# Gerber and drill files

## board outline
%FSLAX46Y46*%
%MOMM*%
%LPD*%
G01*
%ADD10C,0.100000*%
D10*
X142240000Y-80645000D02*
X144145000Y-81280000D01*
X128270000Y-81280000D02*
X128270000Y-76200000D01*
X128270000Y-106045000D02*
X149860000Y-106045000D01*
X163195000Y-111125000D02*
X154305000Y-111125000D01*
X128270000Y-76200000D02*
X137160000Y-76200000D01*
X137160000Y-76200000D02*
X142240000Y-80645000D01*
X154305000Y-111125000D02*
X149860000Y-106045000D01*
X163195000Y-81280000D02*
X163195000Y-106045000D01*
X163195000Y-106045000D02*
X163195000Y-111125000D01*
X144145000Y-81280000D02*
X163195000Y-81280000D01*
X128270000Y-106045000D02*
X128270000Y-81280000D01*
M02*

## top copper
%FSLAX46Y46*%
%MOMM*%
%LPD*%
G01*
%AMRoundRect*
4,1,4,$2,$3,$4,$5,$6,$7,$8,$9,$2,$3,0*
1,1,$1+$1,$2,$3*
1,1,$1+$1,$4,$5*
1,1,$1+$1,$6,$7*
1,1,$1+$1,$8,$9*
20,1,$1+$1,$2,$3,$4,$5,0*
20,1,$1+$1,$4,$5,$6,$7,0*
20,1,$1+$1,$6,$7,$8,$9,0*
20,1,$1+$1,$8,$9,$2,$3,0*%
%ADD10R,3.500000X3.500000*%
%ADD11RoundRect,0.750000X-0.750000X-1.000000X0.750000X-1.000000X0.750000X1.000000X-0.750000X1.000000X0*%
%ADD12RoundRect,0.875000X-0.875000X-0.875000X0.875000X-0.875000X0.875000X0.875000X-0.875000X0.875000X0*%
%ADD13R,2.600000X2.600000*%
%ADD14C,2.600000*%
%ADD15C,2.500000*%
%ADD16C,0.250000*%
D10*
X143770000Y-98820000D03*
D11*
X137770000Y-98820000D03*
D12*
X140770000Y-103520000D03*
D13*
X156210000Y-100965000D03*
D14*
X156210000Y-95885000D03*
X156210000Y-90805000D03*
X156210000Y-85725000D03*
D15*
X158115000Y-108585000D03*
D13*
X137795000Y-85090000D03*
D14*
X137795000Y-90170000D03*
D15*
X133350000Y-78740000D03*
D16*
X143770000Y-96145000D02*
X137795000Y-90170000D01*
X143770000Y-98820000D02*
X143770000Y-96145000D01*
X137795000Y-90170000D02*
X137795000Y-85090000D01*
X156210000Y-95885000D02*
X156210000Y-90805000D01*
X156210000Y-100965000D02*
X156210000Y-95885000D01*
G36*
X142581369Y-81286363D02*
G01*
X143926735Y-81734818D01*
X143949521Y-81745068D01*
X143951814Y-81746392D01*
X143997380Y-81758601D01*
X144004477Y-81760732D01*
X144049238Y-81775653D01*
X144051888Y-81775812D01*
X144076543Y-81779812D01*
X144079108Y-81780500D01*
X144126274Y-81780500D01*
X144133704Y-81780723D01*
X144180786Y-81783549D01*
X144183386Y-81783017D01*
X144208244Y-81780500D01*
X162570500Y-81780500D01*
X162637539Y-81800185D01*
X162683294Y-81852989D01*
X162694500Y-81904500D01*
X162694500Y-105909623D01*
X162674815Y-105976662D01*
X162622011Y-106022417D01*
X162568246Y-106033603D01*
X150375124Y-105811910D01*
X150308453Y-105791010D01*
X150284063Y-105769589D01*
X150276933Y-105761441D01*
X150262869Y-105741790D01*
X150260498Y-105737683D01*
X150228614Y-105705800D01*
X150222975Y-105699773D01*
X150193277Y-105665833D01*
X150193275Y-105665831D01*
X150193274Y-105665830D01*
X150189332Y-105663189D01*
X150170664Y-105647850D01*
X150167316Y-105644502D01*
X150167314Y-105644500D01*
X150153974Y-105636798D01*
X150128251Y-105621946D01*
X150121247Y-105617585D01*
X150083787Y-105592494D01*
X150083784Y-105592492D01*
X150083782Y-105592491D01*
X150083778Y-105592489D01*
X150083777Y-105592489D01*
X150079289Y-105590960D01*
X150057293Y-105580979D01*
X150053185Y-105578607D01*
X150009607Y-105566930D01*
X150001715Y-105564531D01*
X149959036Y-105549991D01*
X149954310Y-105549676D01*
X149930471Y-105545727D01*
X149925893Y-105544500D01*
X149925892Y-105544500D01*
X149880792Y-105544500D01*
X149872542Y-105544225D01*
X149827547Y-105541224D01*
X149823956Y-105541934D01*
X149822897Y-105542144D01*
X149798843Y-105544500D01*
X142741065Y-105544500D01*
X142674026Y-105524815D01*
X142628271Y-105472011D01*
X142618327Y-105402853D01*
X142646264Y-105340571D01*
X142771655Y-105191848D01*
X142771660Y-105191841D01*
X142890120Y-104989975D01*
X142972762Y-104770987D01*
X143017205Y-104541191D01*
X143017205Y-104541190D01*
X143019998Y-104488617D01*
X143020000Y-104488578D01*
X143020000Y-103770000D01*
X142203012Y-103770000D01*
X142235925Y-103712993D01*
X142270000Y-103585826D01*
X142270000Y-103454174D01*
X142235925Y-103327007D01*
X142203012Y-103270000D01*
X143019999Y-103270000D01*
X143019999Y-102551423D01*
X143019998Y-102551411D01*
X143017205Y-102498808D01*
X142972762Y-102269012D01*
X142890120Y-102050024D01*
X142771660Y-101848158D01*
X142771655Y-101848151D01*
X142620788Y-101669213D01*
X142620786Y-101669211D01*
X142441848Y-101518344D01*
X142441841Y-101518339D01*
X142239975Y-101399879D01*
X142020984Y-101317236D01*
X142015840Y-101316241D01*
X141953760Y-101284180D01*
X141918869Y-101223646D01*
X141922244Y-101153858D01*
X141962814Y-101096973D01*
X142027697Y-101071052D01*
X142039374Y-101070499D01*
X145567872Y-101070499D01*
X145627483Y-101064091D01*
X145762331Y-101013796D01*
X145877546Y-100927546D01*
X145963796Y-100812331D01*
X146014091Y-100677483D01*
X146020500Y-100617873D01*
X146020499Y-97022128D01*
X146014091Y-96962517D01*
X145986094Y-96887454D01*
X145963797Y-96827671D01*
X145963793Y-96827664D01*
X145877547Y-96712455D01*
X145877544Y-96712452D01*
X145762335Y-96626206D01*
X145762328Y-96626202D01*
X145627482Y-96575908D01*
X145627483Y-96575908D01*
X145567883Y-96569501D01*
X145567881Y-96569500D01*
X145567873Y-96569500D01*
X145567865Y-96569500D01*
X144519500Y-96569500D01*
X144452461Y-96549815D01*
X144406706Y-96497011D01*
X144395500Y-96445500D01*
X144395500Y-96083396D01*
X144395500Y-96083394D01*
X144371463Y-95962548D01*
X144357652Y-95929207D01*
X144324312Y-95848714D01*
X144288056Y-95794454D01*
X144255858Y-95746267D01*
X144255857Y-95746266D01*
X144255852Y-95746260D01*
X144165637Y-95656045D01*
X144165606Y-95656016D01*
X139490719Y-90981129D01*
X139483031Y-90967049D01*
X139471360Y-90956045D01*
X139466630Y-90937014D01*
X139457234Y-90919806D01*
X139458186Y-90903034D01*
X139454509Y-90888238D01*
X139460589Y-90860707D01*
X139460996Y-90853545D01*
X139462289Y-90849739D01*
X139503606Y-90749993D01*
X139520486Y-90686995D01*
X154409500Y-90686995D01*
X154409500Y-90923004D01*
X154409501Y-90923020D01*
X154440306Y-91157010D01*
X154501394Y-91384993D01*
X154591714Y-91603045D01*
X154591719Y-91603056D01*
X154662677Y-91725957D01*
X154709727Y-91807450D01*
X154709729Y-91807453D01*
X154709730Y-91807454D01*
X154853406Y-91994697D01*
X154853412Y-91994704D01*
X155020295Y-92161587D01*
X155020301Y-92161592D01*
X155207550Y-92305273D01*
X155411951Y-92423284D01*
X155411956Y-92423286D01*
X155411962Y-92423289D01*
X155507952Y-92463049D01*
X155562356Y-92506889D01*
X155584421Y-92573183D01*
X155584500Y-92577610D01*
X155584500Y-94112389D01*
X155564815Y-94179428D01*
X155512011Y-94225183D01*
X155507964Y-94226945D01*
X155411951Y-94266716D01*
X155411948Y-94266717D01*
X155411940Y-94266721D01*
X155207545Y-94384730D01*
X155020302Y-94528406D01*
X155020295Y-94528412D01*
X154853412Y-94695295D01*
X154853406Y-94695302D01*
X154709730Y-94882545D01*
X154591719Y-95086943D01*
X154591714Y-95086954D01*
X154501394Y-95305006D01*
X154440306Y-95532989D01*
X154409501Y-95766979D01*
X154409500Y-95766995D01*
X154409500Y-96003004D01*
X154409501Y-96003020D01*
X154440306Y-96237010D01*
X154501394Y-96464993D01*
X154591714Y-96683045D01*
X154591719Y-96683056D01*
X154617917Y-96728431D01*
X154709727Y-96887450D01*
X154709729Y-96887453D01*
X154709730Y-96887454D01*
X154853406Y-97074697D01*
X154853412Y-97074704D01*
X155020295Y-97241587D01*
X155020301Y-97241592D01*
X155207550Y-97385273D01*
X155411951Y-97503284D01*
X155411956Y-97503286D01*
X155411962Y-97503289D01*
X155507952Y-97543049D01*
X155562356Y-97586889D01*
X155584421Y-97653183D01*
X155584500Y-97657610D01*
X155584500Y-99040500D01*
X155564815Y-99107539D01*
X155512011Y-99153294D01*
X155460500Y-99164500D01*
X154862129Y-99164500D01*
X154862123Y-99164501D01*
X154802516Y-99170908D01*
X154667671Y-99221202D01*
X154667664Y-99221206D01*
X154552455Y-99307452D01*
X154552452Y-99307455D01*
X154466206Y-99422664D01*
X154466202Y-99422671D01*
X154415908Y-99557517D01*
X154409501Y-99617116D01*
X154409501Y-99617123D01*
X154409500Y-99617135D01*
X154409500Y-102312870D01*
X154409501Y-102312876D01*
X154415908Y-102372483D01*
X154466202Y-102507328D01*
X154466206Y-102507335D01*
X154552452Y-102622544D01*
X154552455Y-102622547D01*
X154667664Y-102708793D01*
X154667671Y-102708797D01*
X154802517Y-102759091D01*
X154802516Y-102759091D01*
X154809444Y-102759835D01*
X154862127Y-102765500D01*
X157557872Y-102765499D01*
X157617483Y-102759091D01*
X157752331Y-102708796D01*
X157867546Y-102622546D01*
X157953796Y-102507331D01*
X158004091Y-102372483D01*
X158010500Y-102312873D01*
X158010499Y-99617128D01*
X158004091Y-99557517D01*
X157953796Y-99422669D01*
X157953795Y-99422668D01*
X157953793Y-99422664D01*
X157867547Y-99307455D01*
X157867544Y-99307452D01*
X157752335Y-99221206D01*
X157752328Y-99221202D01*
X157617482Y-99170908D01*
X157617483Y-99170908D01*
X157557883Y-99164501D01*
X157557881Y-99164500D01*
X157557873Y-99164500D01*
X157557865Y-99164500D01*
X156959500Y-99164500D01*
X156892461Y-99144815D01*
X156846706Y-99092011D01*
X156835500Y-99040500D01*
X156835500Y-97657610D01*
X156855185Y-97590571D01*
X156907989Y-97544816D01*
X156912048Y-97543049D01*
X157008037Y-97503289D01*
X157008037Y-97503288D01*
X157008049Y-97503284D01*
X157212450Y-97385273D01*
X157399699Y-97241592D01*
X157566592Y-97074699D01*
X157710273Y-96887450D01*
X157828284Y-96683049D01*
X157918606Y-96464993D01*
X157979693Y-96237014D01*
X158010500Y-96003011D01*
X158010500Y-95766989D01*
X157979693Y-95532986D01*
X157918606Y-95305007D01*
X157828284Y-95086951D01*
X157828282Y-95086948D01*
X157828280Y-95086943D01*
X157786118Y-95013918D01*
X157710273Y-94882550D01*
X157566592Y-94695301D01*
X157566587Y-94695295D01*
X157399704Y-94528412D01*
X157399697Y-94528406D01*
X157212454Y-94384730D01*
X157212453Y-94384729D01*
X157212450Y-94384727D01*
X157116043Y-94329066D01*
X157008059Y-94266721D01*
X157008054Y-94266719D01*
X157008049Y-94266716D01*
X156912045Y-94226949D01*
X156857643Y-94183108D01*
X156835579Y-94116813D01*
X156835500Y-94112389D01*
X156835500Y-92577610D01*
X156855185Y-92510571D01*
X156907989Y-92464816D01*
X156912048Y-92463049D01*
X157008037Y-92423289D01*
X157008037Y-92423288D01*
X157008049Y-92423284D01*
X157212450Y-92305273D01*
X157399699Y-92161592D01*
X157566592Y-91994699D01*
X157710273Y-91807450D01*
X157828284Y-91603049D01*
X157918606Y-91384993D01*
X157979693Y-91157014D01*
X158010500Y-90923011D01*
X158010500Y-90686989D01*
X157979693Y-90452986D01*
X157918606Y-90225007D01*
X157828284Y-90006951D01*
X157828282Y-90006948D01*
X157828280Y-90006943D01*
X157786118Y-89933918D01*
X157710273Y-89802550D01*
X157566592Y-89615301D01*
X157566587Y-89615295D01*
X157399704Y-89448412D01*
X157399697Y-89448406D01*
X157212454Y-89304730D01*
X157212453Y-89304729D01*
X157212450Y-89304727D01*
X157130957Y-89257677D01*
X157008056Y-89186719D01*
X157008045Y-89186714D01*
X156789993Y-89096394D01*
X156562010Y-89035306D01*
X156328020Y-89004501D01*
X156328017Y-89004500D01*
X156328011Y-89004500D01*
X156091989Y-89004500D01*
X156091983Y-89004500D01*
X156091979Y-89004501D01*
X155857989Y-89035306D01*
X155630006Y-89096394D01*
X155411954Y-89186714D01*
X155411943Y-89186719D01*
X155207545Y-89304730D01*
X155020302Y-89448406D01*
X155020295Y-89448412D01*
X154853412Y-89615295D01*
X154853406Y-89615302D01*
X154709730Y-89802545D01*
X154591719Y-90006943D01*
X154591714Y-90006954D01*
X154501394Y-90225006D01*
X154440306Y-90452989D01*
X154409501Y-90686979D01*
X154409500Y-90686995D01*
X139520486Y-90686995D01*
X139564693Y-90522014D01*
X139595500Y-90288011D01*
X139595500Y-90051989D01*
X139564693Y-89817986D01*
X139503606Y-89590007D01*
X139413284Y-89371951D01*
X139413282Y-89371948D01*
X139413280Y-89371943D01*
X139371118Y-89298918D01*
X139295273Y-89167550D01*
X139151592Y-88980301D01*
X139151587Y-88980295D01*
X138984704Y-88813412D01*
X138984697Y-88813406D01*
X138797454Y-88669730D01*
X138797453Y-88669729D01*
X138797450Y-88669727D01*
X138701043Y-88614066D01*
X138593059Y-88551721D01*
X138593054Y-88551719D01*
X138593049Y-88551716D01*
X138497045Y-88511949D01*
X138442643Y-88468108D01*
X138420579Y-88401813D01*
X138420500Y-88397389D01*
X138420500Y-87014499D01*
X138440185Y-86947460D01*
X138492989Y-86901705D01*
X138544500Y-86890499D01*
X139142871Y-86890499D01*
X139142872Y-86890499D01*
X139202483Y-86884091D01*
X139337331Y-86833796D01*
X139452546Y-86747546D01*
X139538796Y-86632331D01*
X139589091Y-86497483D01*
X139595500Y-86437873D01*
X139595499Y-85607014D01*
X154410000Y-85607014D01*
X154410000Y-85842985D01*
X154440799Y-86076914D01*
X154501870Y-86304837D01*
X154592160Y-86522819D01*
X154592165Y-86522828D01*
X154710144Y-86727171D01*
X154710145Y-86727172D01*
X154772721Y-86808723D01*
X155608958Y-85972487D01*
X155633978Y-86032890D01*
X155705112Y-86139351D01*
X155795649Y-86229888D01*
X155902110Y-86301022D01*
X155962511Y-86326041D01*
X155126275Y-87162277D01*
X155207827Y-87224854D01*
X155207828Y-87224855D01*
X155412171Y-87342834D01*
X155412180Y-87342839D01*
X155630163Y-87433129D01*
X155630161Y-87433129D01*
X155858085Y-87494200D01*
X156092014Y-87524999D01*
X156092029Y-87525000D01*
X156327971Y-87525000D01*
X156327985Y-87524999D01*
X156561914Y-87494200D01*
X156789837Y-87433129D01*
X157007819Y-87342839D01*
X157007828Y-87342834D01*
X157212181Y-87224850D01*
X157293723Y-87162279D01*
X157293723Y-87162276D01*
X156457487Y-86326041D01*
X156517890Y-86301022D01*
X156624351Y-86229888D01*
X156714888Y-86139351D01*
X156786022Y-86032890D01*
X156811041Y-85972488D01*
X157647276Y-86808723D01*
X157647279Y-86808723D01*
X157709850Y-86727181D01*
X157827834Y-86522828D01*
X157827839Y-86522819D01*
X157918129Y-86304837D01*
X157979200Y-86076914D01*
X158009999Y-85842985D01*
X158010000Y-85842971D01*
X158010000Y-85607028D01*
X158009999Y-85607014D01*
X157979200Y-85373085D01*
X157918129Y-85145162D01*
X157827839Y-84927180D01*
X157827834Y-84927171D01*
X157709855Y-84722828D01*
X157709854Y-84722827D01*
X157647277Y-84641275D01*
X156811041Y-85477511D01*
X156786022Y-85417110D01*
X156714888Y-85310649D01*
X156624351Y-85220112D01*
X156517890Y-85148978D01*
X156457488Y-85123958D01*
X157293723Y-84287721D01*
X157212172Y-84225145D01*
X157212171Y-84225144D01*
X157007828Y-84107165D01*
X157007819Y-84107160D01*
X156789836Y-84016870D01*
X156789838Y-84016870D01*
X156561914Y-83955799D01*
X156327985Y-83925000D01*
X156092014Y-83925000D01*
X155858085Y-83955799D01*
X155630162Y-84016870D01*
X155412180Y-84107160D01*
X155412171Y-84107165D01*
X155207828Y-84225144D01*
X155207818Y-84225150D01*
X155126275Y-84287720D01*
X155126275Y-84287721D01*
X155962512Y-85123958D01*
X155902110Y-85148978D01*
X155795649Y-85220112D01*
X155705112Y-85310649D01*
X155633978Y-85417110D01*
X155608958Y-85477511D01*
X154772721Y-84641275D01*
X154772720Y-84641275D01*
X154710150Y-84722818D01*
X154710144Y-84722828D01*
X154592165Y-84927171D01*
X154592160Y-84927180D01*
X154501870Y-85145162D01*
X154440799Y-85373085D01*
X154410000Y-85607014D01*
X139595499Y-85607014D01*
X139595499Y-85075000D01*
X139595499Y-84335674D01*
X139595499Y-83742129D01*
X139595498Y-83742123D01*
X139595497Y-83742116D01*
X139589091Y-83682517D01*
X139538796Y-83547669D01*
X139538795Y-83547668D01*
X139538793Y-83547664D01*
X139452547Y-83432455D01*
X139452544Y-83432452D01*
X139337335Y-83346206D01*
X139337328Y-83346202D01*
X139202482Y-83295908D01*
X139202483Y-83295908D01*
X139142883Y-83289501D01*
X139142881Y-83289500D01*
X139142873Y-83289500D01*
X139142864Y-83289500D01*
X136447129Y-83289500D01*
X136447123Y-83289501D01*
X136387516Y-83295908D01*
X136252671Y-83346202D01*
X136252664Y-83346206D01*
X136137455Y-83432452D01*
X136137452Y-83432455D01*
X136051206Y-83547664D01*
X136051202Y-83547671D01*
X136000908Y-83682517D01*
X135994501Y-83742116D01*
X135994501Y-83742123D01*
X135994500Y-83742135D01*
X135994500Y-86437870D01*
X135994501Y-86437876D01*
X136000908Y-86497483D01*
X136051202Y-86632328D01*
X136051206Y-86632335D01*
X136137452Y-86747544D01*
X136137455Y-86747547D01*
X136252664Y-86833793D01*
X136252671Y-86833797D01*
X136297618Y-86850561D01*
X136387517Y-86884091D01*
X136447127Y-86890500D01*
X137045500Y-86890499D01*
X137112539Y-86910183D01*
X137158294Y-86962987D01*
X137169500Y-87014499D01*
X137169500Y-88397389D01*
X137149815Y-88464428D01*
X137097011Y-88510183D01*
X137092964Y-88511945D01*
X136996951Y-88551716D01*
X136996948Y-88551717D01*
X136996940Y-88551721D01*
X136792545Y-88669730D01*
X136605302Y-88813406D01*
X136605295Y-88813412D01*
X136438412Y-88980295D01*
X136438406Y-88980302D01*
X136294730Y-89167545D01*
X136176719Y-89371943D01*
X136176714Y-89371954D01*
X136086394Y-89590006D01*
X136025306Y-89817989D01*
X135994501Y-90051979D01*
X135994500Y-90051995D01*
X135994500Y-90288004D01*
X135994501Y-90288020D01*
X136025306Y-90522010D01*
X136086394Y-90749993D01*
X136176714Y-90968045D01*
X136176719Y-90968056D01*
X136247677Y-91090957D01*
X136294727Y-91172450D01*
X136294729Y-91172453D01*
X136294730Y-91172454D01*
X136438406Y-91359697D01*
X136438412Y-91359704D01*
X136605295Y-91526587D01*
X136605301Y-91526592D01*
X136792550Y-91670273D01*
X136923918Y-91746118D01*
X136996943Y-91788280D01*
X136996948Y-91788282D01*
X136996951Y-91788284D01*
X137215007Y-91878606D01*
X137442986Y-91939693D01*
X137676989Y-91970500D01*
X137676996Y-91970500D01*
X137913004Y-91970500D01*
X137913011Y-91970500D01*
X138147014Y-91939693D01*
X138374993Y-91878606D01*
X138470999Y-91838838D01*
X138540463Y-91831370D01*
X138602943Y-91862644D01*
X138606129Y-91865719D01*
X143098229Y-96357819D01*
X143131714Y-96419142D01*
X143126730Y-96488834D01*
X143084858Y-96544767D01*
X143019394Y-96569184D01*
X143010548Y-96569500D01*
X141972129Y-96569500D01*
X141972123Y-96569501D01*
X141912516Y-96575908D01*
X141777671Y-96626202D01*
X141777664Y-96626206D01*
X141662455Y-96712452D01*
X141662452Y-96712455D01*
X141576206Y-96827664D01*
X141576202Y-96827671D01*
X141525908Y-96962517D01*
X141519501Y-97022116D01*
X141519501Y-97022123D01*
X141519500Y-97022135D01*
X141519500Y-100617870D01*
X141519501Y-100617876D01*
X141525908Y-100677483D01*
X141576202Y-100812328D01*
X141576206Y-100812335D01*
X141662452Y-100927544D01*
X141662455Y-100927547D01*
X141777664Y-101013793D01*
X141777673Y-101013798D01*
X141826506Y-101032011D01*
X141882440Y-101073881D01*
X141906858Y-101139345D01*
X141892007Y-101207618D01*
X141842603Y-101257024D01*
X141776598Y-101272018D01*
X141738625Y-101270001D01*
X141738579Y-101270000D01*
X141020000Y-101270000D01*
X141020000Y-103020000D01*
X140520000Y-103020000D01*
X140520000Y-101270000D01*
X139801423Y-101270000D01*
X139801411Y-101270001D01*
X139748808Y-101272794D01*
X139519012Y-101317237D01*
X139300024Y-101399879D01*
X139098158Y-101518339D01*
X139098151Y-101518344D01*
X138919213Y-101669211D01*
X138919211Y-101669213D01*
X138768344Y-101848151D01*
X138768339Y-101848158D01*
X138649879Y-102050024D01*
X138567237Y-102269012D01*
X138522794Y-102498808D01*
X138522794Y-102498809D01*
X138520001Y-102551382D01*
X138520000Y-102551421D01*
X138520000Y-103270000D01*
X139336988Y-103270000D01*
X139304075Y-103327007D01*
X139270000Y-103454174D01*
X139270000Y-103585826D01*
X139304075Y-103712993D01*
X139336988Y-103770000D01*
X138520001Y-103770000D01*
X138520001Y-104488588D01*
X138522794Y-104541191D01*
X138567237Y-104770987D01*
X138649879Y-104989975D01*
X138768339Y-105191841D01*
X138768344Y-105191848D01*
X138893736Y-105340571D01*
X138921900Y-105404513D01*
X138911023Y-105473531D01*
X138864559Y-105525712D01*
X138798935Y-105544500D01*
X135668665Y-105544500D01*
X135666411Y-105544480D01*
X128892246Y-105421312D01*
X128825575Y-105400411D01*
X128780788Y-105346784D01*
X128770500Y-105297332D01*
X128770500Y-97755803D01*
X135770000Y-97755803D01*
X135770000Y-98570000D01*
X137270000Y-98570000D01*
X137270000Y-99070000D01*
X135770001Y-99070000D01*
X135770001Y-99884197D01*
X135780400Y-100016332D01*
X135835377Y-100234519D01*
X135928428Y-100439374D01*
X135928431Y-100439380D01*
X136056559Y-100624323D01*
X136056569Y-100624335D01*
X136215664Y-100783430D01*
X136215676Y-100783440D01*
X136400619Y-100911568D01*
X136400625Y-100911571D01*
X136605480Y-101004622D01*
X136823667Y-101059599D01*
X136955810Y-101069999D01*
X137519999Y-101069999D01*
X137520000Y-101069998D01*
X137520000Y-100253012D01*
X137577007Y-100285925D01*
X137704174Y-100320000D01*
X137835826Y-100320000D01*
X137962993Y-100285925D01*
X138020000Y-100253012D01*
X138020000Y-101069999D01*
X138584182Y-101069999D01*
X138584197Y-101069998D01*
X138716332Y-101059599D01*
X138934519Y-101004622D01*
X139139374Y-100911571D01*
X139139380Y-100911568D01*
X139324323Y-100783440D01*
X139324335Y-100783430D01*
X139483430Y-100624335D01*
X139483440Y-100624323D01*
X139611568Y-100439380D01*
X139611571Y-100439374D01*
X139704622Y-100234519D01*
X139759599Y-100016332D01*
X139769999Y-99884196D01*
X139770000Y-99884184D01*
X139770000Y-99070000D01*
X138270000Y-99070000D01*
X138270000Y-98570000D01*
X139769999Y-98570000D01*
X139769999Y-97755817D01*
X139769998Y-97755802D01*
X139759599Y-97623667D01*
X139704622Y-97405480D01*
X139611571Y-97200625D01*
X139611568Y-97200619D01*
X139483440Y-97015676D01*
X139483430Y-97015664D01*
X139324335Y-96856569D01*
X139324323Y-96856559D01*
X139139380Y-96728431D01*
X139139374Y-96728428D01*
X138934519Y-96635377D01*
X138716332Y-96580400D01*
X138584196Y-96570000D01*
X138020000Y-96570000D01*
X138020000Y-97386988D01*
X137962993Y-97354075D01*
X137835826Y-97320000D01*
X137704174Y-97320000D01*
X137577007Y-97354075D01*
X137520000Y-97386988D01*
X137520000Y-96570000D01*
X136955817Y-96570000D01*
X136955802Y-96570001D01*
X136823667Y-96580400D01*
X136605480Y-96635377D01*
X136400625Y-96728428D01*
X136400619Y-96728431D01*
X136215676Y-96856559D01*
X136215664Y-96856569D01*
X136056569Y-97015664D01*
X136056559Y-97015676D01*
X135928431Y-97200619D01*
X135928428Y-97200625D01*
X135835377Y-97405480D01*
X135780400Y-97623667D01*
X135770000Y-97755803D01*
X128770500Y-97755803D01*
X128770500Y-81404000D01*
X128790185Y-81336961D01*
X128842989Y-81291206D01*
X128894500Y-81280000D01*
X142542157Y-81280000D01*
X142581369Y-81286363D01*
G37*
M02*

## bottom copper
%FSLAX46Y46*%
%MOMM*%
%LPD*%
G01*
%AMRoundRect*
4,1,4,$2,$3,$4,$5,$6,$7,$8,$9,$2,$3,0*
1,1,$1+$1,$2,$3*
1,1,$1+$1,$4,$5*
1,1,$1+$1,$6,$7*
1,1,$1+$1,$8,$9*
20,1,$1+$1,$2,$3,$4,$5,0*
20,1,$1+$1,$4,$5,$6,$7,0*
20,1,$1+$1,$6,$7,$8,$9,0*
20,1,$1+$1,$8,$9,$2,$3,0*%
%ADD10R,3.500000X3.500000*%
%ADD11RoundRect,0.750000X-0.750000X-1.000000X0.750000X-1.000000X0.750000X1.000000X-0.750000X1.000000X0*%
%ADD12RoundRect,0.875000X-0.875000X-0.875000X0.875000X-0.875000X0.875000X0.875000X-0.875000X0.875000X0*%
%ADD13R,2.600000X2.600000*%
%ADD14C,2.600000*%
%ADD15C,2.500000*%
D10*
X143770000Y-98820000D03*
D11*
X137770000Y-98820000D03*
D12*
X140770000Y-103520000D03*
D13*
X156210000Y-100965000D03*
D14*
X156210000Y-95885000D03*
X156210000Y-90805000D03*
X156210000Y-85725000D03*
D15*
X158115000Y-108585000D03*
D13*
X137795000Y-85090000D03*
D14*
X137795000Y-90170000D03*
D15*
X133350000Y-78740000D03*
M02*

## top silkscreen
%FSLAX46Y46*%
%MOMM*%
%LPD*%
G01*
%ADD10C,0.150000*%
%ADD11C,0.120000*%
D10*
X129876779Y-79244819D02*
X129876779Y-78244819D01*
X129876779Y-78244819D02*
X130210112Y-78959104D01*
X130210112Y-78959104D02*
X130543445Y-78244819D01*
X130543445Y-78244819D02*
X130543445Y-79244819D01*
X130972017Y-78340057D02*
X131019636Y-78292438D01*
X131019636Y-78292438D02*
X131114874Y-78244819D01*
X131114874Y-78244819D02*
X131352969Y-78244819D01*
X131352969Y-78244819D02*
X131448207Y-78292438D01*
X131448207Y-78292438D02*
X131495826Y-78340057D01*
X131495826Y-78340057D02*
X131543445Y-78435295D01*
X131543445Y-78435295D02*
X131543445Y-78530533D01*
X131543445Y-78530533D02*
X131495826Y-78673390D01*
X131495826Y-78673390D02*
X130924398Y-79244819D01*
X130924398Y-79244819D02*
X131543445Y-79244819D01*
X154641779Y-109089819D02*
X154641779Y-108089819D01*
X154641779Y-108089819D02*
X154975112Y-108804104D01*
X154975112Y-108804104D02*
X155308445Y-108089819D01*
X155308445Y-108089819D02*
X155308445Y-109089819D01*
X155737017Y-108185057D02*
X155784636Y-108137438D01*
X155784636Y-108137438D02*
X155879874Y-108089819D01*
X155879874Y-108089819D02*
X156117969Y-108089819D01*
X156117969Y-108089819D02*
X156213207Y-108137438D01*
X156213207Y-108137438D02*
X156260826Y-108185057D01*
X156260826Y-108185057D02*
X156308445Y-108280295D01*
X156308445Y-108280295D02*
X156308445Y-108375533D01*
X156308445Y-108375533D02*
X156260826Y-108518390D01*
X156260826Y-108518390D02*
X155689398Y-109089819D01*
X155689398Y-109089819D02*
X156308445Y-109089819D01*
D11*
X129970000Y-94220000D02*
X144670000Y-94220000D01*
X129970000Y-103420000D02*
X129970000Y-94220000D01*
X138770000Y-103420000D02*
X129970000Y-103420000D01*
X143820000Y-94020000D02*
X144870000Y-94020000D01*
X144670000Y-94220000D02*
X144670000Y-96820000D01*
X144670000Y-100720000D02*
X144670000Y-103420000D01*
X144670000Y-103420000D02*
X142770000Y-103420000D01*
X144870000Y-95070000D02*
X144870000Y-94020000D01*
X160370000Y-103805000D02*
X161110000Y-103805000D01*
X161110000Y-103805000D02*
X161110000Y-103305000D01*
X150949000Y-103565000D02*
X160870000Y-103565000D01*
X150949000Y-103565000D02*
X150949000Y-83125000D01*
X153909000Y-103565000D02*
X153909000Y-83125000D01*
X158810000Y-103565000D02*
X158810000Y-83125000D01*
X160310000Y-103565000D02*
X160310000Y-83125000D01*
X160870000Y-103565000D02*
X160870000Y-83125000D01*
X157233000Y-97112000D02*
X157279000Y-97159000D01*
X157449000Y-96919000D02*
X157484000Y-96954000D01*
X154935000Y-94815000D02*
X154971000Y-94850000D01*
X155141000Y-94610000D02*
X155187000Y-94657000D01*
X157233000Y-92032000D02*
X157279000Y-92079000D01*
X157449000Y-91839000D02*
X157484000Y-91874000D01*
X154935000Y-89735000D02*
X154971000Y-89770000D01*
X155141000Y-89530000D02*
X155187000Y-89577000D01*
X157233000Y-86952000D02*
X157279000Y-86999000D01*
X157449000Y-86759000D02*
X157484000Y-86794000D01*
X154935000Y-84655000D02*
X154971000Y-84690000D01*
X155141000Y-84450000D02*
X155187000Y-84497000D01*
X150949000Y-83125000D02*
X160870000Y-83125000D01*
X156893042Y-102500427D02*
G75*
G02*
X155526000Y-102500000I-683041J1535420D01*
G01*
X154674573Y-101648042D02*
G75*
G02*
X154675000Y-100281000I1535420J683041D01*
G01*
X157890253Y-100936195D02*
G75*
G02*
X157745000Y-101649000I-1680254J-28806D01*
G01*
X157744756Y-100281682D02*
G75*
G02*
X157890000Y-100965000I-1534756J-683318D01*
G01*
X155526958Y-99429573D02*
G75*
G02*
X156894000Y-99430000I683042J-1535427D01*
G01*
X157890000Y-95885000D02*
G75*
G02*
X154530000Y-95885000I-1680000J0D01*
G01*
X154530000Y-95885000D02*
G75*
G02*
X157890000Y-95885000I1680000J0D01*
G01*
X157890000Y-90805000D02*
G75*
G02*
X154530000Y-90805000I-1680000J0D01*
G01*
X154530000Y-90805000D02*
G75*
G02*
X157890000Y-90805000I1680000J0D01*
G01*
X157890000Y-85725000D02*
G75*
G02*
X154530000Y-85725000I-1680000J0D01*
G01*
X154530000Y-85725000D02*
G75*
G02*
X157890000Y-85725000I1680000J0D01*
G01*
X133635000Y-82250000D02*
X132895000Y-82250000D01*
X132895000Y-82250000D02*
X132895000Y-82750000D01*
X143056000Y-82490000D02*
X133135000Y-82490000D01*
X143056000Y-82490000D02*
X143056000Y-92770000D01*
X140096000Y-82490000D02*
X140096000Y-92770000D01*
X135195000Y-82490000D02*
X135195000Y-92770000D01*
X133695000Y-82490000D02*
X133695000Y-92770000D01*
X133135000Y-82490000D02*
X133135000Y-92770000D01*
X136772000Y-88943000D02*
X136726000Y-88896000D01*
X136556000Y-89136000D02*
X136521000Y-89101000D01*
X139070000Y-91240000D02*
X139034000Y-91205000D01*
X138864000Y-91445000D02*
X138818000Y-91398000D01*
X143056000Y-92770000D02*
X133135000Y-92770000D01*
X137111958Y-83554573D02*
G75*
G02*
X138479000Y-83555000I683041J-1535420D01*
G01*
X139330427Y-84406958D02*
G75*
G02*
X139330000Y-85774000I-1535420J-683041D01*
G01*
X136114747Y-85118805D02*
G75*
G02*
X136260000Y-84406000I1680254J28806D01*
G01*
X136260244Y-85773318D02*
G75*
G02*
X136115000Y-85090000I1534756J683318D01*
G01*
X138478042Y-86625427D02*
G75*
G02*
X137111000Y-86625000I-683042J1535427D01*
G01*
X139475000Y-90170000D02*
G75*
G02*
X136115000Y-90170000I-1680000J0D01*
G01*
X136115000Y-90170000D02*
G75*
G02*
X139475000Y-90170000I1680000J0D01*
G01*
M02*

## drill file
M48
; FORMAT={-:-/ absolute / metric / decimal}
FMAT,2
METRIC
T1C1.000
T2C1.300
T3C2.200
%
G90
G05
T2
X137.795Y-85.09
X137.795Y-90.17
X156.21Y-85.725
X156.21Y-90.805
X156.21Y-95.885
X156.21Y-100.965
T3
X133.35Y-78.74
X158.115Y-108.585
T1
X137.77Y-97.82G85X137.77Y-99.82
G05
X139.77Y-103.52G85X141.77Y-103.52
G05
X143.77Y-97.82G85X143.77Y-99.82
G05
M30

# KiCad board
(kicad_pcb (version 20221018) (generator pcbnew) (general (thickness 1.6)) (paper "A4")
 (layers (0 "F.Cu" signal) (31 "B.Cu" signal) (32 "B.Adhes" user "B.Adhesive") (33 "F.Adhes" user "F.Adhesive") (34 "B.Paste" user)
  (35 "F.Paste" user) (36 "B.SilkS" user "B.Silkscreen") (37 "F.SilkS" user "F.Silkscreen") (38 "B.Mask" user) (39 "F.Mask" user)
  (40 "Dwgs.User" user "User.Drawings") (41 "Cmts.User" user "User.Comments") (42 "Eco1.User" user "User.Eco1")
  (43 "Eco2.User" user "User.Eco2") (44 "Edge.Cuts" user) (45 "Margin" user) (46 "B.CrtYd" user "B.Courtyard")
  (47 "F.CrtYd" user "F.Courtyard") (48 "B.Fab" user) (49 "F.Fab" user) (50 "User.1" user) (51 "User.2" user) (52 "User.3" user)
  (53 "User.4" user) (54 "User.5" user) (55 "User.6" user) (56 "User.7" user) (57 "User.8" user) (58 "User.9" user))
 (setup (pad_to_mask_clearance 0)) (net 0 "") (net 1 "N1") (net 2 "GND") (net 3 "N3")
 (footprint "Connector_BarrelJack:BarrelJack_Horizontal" (layer "F.Cu") (at 143.77 98.82)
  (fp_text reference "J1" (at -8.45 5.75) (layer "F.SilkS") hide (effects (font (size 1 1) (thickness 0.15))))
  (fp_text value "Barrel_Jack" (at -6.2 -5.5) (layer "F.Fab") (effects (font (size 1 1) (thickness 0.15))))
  (fp_line (start -13.8 -4.6) (end 0.9 -4.6) (stroke (width 0.12) (type solid)) (layer "F.SilkS"))
  (fp_line (start -13.8 4.6) (end -13.8 -4.6) (stroke (width 0.12) (type solid)) (layer "F.SilkS"))
  (fp_line (start -5 4.6) (end -13.8 4.6) (stroke (width 0.12) (type solid)) (layer "F.SilkS"))
  (fp_line (start 0.05 -4.8) (end 1.1 -4.8) (stroke (width 0.12) (type solid)) (layer "F.SilkS"))
  (fp_line (start 0.9 -4.6) (end 0.9 -2) (stroke (width 0.12) (type solid)) (layer "F.SilkS"))
  (fp_line (start 0.9 1.9) (end 0.9 4.6) (stroke (width 0.12) (type solid)) (layer "F.SilkS"))
  (fp_line (start 0.9 4.6) (end -1 4.6) (stroke (width 0.12) (type solid)) (layer "F.SilkS"))
  (fp_line (start 1.1 -3.75) (end 1.1 -4.8) (stroke (width 0.12) (type solid)) (layer "F.SilkS"))
  (pad "1" thru_hole rect (at 0 0) (size 3.5 3.5) (drill oval 1 3) (layers "*.Cu" "*.Mask") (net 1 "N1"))
  (pad "2" thru_hole roundrect (at -6 0) (size 3 3.5) (drill oval 1 3) (layers "*.Cu" "*.Mask") (roundrect_rratio 0.25) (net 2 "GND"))
  (pad "3" thru_hole roundrect (at -3 4.7) (size 3.5 3.5) (drill oval 3 1) (layers "*.Cu" "*.Mask") (roundrect_rratio 0.25) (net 2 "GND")))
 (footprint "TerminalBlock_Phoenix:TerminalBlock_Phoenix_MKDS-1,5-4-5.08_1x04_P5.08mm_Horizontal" (layer "F.Cu") (at 156.21 100.965 90)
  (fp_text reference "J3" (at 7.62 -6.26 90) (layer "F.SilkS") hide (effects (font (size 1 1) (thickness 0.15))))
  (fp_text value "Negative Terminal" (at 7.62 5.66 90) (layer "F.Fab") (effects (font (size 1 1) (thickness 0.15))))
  (fp_line (start -2.84 4.16) (end -2.84 4.9) (stroke (width 0.12) (type solid)) (layer "F.SilkS"))
  (fp_line (start -2.84 4.9) (end -2.34 4.9) (stroke (width 0.12) (type solid)) (layer "F.SilkS"))
  (fp_line (start -2.6 -5.261) (end -2.6 4.66) (stroke (width 0.12) (type solid)) (layer "F.SilkS"))
  (fp_line (start -2.6 -5.261) (end 17.84 -5.261) (stroke (width 0.12) (type solid)) (layer "F.SilkS"))
  (fp_line (start -2.6 -2.301) (end 17.84 -2.301) (stroke (width 0.12) (type solid)) (layer "F.SilkS"))
  (fp_line (start -2.6 2.6) (end 17.84 2.6) (stroke (width 0.12) (type solid)) (layer "F.SilkS"))
  (fp_line (start -2.6 4.1) (end 17.84 4.1) (stroke (width 0.12) (type solid)) (layer "F.SilkS"))
  (fp_line (start -2.6 4.66) (end 17.84 4.66) (stroke (width 0.12) (type solid)) (layer "F.SilkS"))
  (fp_line (start 3.853 1.023) (end 3.806 1.069) (stroke (width 0.12) (type solid)) (layer "F.SilkS"))
  (fp_line (start 4.046 1.239) (end 4.011 1.274) (stroke (width 0.12) (type solid)) (layer "F.SilkS"))
  (fp_line (start 6.15 -1.275) (end 6.115 -1.239) (stroke (width 0.12) (type solid)) (layer "F.SilkS"))
  (fp_line (start 6.355 -1.069) (end 6.308 -1.023) (stroke (width 0.12) (type solid)) (layer "F.SilkS"))
  (fp_line (start 8.933 1.023) (end 8.886 1.069) (stroke (width 0.12) (type solid)) (layer "F.SilkS"))
  (fp_line (start 9.126 1.239) (end 9.091 1.274) (stroke (width 0.12) (type solid)) (layer "F.SilkS"))
  (fp_line (start 11.23 -1.275) (end 11.195 -1.239) (stroke (width 0.12) (type solid)) (layer "F.SilkS"))
  (fp_line (start 11.435 -1.069) (end 11.388 -1.023) (stroke (width 0.12) (type solid)) (layer "F.SilkS"))
  (fp_line (start 14.013 1.023) (end 13.966 1.069) (stroke (width 0.12) (type solid)) (layer "F.SilkS"))
  (fp_line (start 14.206 1.239) (end 14.171 1.274) (stroke (width 0.12) (type solid)) (layer "F.SilkS"))
  (fp_line (start 16.31 -1.275) (end 16.275 -1.239) (stroke (width 0.12) (type solid)) (layer "F.SilkS"))
  (fp_line (start 16.515 -1.069) (end 16.468 -1.023) (stroke (width 0.12) (type solid)) (layer "F.SilkS"))
  (fp_line (start 17.84 -5.261) (end 17.84 4.66) (stroke (width 0.12) (type solid)) (layer "F.SilkS"))
  (fp_arc (start -1.535427 0.683042) (mid -1.680501 -0.000524) (end -1.535 -0.684) (stroke (width 0.12) (type solid)) (layer "F.SilkS"))
  (fp_arc (start -0.683042 -1.535427) (mid 0.000524 -1.680501) (end 0.684 -1.535) (stroke (width 0.12) (type solid)) (layer "F.SilkS"))
  (fp_arc (start 0.028805 1.680253) (mid -0.335551 1.646659) (end -0.684 1.535) (stroke (width 0.12) (type solid)) (layer "F.SilkS"))
  (fp_arc (start 0.683318 1.534756) (mid 0.349292 1.643288) (end 0 1.68) (stroke (width 0.12) (type solid)) (layer "F.SilkS"))
  (fp_arc (start 1.535427 -0.683042) (mid 1.680501 0.000524) (end 1.535 0.684) (stroke (width 0.12) (type solid)) (layer "F.SilkS"))
  (fp_circle (center 5.08 0) (end 6.76 0) (stroke (width 0.12) (type solid)) (fill none) (layer "F.SilkS"))
  (fp_circle (center 10.16 0) (end 11.84 0) (stroke (width 0.12) (type solid)) (fill none) (layer "F.SilkS"))
  (fp_circle (center 15.24 0) (end 16.92 0) (stroke (width 0.12) (type solid)) (fill none) (layer "F.SilkS"))
  (pad "1" thru_hole rect (at 0 0 90) (size 2.6 2.6) (drill 1.3) (layers "*.Cu" "*.Mask") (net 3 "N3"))
  (pad "2" thru_hole circle (at 5.08 0 90) (size 2.6 2.6) (drill 1.3) (layers "*.Cu" "*.Mask") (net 3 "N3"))
  (pad "3" thru_hole circle (at 10.16 0 90) (size 2.6 2.6) (drill 1.3) (layers "*.Cu" "*.Mask") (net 3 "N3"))
  (pad "4" thru_hole circle (at 15.24 0 90) (size 2.6 2.6) (drill 1.3) (layers "*.Cu" "*.Mask") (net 2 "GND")))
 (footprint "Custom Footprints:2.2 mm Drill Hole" (layer "F.Cu") (at 158.115 108.585)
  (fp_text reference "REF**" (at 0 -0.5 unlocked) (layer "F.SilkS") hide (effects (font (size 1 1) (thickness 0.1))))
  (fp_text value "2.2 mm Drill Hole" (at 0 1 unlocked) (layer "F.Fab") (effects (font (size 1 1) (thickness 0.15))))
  (pad "" np_thru_hole circle (at 0 0) (size 2.5 2.5) (drill 2.2) (layers "F&B.Cu" "*.Mask")))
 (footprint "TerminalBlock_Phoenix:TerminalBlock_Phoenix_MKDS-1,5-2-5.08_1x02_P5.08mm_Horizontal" (layer "F.Cu") (at 137.795 85.09 -90)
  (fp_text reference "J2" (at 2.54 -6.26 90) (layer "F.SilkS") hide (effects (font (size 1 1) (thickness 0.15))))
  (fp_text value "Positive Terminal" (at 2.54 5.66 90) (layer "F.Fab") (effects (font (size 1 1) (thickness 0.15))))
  (fp_line (start -2.84 4.16) (end -2.84 4.9) (stroke (width 0.12) (type solid)) (layer "F.SilkS"))
  (fp_line (start -2.84 4.9) (end -2.34 4.9) (stroke (width 0.12) (type solid)) (layer "F.SilkS"))
  (fp_line (start -2.6 -5.261) (end -2.6 4.66) (stroke (width 0.12) (type solid)) (layer "F.SilkS"))
  (fp_line (start -2.6 -5.261) (end 7.68 -5.261) (stroke (width 0.12) (type solid)) (layer "F.SilkS"))
  (fp_line (start -2.6 -2.301) (end 7.68 -2.301) (stroke (width 0.12) (type solid)) (layer "F.SilkS"))
  (fp_line (start -2.6 2.6) (end 7.68 2.6) (stroke (width 0.12) (type solid)) (layer "F.SilkS"))
  (fp_line (start -2.6 4.1) (end 7.68 4.1) (stroke (width 0.12) (type solid)) (layer "F.SilkS"))
  (fp_line (start -2.6 4.66) (end 7.68 4.66) (stroke (width 0.12) (type solid)) (layer "F.SilkS"))
  (fp_line (start 3.853 1.023) (end 3.806 1.069) (stroke (width 0.12) (type solid)) (layer "F.SilkS"))
  (fp_line (start 4.046 1.239) (end 4.011 1.274) (stroke (width 0.12) (type solid)) (layer "F.SilkS"))
  (fp_line (start 6.15 -1.275) (end 6.115 -1.239) (stroke (width 0.12) (type solid)) (layer "F.SilkS"))
  (fp_line (start 6.355 -1.069) (end 6.308 -1.023) (stroke (width 0.12) (type solid)) (layer "F.SilkS"))
  (fp_line (start 7.68 -5.261) (end 7.68 4.66) (stroke (width 0.12) (type solid)) (layer "F.SilkS"))
  (fp_arc (start -1.535427 0.683042) (mid -1.680501 -0.000524) (end -1.535 -0.684) (stroke (width 0.12) (type solid)) (layer "F.SilkS"))
  (fp_arc (start -0.683042 -1.535427) (mid 0.000524 -1.680501) (end 0.684 -1.535) (stroke (width 0.12) (type solid)) (layer "F.SilkS"))
  (fp_arc (start 0.028805 1.680253) (mid -0.335551 1.646659) (end -0.684 1.535) (stroke (width 0.12) (type solid)) (layer "F.SilkS"))
  (fp_arc (start 0.683318 1.534756) (mid 0.349292 1.643288) (end 0 1.68) (stroke (width 0.12) (type solid)) (layer "F.SilkS"))
  (fp_arc (start 1.535427 -0.683042) (mid 1.680501 0.000524) (end 1.535 0.684) (stroke (width 0.12) (type solid)) (layer "F.SilkS"))
  (fp_circle (center 5.08 0) (end 6.76 0) (stroke (width 0.12) (type solid)) (fill none) (layer "F.SilkS"))
  (pad "1" thru_hole rect (at 0 0 270) (size 2.6 2.6) (drill 1.3) (layers "*.Cu" "*.Mask") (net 1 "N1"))
  (pad "2" thru_hole circle (at 5.08 0 270) (size 2.6 2.6) (drill 1.3) (layers "*.Cu" "*.Mask") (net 1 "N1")))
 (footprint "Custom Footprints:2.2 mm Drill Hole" (layer "F.Cu") (at 133.35 78.74)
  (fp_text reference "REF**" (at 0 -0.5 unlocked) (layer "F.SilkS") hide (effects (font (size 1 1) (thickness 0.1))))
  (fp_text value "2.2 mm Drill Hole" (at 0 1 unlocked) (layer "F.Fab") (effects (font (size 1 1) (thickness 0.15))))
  (pad "" np_thru_hole circle (at 0 0) (size 2.5 2.5) (drill 2.2) (layers "F&B.Cu" "*.Mask")))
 (gr_line (start 142.24 80.645) (end 144.145 81.28) (stroke (width 0.1) (type default)) (layer "Edge.Cuts"))
 (gr_line (start 128.27 81.28) (end 128.27 76.2) (stroke (width 0.1) (type default)) (layer "Edge.Cuts"))
 (gr_line (start 128.27 106.045) (end 149.86 106.045) (stroke (width 0.1) (type default)) (layer "Edge.Cuts"))
 (gr_line (start 163.195 111.125) (end 154.305 111.125) (stroke (width 0.1) (type default)) (layer "Edge.Cuts"))
 (gr_line (start 128.27 76.2) (end 137.16 76.2) (stroke (width 0.1) (type default)) (layer "Edge.Cuts"))
 (gr_line (start 137.16 76.2) (end 142.24 80.645) (stroke (width 0.1) (type default)) (layer "Edge.Cuts"))
 (gr_line (start 154.305 111.125) (end 149.86 106.045) (stroke (width 0.1) (type default)) (layer "Edge.Cuts"))
 (gr_line (start 163.195 81.28) (end 163.195 106.045) (stroke (width 0.1) (type default)) (layer "Edge.Cuts"))
 (gr_line (start 163.195 106.045) (end 163.195 111.125) (stroke (width 0.1) (type default)) (layer "Edge.Cuts"))
 (gr_line (start 144.145 81.28) (end 163.195 81.28) (stroke (width 0.1) (type default)) (layer "Edge.Cuts"))
 (gr_line (start 128.27 106.045) (end 128.27 81.28) (stroke (width 0.1) (type default)) (layer "Edge.Cuts"))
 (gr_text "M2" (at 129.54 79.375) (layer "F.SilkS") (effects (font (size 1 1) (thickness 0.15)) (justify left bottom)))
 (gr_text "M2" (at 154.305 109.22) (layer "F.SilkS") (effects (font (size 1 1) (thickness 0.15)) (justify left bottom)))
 (segment (start 143.77 96.145) (end 137.795 90.17) (width 0.25) (layer "F.Cu") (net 1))
 (segment (start 143.77 98.82) (end 143.77 96.145) (width 0.25) (layer "F.Cu") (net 1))
 (segment (start 137.795 90.17) (end 137.795 85.09) (width 0.25) (layer "F.Cu") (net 1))
 (segment (start 156.21 95.885) (end 156.21 90.805) (width 0.25) (layer "F.Cu") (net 3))
 (segment (start 156.21 100.965) (end 156.21 95.885) (width 0.25) (layer "F.Cu") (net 3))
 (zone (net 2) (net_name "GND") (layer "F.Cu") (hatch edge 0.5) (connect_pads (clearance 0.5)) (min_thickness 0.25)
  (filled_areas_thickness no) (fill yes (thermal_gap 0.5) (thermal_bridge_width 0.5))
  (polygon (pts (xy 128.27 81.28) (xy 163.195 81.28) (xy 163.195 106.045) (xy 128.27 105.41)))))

